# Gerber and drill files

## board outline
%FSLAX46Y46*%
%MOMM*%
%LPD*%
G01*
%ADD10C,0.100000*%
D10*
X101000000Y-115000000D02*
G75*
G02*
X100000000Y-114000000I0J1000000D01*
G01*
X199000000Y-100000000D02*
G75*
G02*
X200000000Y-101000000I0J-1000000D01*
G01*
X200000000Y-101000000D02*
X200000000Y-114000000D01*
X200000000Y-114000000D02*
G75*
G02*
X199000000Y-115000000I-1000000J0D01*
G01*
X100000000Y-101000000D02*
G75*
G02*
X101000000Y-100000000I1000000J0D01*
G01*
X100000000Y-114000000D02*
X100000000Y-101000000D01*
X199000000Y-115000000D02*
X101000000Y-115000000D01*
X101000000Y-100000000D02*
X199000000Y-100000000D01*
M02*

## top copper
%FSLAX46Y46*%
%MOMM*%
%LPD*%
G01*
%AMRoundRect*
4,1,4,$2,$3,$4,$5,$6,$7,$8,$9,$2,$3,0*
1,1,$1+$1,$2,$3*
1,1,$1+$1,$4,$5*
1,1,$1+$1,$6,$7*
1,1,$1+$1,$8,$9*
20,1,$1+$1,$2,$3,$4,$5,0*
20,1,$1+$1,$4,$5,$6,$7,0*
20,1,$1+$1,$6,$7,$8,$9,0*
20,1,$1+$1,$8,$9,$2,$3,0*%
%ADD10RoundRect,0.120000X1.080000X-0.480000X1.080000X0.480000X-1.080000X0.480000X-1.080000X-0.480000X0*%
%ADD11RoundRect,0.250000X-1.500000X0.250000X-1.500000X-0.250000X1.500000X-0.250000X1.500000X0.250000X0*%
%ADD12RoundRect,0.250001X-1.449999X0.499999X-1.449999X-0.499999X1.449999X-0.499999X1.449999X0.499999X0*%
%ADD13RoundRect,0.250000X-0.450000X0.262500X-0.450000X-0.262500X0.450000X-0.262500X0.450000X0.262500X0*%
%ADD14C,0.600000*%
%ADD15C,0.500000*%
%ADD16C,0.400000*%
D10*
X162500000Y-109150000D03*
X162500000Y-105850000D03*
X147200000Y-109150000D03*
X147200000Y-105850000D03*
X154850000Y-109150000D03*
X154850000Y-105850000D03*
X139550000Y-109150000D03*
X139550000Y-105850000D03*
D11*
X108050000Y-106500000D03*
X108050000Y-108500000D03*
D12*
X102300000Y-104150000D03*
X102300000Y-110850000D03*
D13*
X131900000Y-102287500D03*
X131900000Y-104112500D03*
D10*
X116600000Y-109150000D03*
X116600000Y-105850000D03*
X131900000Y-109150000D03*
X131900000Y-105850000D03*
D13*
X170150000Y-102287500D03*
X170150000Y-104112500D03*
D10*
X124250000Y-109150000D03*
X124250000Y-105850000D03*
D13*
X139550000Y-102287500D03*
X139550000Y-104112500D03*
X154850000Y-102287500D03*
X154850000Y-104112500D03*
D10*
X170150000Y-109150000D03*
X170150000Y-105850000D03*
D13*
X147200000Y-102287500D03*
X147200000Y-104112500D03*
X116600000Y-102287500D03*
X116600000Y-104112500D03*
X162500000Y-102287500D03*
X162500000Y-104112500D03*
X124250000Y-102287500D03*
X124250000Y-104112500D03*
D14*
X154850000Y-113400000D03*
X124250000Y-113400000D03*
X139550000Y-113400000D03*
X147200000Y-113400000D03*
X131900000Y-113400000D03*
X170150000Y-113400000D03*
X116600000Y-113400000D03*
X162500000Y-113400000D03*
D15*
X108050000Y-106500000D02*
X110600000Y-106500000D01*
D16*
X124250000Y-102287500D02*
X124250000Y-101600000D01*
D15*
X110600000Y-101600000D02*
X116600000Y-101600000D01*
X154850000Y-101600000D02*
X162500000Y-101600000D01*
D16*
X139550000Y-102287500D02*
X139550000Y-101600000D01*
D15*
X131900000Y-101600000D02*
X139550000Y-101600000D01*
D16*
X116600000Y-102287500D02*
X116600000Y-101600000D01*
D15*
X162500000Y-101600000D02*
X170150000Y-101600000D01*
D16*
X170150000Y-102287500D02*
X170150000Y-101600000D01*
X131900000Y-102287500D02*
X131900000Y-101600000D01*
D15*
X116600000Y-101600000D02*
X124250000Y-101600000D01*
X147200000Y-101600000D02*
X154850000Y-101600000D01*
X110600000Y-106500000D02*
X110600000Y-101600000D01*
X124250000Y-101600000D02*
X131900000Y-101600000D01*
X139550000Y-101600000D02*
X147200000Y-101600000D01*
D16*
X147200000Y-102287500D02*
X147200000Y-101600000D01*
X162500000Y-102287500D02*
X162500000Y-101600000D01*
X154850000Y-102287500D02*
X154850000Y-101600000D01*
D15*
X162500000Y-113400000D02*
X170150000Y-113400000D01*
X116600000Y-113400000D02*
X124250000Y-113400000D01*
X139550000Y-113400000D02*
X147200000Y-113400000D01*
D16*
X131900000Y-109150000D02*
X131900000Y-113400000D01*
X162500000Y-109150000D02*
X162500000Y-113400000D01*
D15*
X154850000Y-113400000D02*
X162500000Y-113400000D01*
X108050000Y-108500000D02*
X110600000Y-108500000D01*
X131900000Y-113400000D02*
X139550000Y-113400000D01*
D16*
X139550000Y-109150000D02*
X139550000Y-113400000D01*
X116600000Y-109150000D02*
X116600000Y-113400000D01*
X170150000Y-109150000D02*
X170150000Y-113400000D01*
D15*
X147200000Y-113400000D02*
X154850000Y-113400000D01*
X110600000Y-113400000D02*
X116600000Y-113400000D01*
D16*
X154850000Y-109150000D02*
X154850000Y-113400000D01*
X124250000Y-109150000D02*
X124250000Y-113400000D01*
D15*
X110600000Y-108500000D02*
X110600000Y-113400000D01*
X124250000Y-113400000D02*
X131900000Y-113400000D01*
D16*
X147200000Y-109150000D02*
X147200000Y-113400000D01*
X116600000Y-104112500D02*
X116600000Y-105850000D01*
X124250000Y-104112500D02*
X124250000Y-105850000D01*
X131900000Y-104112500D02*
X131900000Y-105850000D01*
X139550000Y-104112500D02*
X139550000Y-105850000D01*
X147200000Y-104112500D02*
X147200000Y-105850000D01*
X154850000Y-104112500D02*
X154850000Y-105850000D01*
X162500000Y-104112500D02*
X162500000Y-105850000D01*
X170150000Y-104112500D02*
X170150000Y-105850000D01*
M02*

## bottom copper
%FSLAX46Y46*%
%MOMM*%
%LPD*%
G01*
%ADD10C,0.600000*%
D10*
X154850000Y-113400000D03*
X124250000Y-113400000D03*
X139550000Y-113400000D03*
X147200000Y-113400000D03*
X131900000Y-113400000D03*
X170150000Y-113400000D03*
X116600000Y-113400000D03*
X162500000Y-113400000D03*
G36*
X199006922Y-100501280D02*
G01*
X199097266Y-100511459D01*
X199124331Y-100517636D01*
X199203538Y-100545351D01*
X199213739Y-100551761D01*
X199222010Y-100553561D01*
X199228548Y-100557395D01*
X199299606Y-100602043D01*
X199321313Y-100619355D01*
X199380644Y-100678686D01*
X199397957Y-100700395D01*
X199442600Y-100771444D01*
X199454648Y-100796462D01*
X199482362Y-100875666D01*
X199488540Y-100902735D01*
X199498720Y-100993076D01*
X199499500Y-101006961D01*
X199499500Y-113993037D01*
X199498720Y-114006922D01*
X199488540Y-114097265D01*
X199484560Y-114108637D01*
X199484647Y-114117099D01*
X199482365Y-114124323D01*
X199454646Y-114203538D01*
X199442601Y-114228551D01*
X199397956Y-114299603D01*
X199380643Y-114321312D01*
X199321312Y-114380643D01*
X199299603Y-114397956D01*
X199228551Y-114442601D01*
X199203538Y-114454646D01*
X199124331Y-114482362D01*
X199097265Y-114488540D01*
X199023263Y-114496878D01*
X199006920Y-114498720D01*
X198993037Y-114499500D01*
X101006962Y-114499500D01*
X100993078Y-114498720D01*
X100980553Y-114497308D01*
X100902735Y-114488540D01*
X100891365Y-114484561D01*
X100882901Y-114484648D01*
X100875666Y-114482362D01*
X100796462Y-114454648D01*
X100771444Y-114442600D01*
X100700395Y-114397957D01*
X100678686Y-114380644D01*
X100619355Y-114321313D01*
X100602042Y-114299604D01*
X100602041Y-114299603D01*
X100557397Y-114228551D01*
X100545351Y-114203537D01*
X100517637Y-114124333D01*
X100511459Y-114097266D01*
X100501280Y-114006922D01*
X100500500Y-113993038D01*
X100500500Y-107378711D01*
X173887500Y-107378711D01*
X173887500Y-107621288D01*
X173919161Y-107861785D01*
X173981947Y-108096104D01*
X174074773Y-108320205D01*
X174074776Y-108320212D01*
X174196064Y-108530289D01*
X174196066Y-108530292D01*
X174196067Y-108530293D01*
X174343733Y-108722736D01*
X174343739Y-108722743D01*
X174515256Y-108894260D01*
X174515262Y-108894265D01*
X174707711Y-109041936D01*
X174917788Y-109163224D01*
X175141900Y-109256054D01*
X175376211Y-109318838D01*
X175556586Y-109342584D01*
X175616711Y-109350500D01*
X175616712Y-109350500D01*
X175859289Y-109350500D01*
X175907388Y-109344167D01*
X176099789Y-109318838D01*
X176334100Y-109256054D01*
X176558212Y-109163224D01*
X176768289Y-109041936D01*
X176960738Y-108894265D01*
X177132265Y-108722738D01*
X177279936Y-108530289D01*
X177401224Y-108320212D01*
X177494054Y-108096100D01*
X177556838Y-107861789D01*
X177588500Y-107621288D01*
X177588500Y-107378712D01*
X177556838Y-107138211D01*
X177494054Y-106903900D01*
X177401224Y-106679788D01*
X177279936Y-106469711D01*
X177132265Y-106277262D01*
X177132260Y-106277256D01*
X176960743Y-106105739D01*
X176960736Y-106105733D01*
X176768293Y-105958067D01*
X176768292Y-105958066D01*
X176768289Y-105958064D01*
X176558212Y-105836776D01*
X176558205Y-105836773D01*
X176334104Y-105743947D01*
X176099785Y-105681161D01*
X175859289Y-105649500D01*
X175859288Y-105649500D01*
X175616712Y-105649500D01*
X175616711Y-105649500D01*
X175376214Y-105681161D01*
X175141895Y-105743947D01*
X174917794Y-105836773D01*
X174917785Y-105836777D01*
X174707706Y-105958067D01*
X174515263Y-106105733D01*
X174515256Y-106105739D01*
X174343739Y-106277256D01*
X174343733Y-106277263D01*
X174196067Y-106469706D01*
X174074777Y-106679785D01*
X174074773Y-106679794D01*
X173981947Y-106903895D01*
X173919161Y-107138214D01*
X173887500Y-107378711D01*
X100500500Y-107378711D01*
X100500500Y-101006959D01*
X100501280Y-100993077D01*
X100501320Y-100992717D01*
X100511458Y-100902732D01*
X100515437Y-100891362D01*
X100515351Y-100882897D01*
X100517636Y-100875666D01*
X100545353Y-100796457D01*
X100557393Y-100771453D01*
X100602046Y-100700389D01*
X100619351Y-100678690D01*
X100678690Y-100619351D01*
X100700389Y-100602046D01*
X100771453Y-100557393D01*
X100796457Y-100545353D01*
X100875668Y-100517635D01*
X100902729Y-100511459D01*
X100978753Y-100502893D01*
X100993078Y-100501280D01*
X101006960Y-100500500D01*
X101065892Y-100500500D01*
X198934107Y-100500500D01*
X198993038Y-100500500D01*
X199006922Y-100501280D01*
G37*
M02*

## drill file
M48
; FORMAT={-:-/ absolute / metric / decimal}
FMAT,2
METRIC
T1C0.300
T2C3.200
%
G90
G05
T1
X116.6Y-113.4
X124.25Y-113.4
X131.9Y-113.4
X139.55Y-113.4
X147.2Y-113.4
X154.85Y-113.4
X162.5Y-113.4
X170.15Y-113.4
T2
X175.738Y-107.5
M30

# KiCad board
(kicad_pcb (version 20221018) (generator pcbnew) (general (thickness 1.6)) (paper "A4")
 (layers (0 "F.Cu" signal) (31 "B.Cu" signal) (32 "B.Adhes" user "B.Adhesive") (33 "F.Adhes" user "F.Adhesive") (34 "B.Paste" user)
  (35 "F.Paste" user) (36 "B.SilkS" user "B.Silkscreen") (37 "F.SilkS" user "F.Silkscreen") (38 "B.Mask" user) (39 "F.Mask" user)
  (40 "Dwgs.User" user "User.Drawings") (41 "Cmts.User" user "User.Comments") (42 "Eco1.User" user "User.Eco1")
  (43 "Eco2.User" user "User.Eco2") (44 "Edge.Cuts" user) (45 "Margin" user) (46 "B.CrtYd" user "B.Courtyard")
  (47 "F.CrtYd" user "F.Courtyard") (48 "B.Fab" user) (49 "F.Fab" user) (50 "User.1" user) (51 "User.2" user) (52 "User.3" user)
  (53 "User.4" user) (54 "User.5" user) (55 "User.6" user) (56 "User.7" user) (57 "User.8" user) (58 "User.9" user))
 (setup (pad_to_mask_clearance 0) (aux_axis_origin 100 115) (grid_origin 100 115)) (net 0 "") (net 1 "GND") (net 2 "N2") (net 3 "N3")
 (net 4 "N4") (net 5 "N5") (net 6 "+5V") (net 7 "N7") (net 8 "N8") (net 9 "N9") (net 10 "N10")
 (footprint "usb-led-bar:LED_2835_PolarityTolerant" (layer "F.Cu") (at 162.5 107.5 90)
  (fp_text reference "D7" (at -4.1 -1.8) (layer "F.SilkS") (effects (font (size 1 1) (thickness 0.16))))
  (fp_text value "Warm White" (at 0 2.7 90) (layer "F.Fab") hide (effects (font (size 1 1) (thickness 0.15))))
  (pad "1" smd roundrect (at -1.65 0 90) (size 1.2 2.4) (layers "F.Cu" "F.Paste" "F.Mask") (roundrect_rratio 0.1) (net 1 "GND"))
  (pad "2" smd roundrect (at 1.65 0 90) (size 1.2 2.4) (layers "F.Cu" "F.Paste" "F.Mask") (roundrect_rratio 0.1) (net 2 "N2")))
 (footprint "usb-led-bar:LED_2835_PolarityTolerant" (layer "F.Cu") (at 147.2 107.5 90)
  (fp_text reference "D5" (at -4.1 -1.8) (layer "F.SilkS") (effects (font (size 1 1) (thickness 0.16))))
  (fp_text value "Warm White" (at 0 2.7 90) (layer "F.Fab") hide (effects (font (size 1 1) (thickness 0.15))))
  (pad "1" smd roundrect (at -1.65 0 90) (size 1.2 2.4) (layers "F.Cu" "F.Paste" "F.Mask") (roundrect_rratio 0.1) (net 1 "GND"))
  (pad "2" smd roundrect (at 1.65 0 90) (size 1.2 2.4) (layers "F.Cu" "F.Paste" "F.Mask") (roundrect_rratio 0.1) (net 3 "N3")))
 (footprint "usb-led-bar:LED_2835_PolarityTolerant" (layer "F.Cu") (at 154.85 107.5 90)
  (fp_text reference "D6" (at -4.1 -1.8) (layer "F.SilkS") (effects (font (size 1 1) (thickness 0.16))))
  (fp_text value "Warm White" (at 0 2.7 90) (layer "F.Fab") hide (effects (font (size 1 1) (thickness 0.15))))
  (pad "1" smd roundrect (at -1.65 0 90) (size 1.2 2.4) (layers "F.Cu" "F.Paste" "F.Mask") (roundrect_rratio 0.1) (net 1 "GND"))
  (pad "2" smd roundrect (at 1.65 0 90) (size 1.2 2.4) (layers "F.Cu" "F.Paste" "F.Mask") (roundrect_rratio 0.1) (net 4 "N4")))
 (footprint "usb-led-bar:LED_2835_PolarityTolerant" (layer "F.Cu") (at 139.55 107.5 90)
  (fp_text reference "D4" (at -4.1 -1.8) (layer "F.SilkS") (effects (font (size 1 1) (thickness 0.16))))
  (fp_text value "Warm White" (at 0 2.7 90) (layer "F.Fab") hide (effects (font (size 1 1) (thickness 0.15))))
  (pad "1" smd roundrect (at -1.65 0 90) (size 1.2 2.4) (layers "F.Cu" "F.Paste" "F.Mask") (roundrect_rratio 0.1) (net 1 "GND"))
  (pad "2" smd roundrect (at 1.65 0 90) (size 1.2 2.4) (layers "F.Cu" "F.Paste" "F.Mask") (roundrect_rratio 0.1) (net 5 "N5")))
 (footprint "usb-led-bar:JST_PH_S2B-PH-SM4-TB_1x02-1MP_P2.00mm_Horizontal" (layer "F.Cu") (at 105.2 107.5 -90)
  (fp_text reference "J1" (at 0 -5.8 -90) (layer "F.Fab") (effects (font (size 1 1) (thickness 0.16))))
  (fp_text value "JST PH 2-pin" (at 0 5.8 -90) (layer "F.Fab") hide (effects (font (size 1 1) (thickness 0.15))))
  (pad "1" smd roundrect (at -1 -2.85 270) (size 1 3.5) (layers "F.Cu" "F.Paste" "F.Mask") (roundrect_rratio 0.25) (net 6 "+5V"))
  (pad "2" smd roundrect (at 1 -2.85 270) (size 1 3.5) (layers "F.Cu" "F.Paste" "F.Mask") (roundrect_rratio 0.25) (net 1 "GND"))
  (pad "MP" smd roundrect (at -3.35 2.9 270) (size 1.5 3.4) (layers "F.Cu" "F.Paste" "F.Mask") (roundrect_rratio 0.166667))
  (pad "MP" smd roundrect (at 3.35 2.9 270) (size 1.5 3.4) (layers "F.Cu" "F.Paste" "F.Mask") (roundrect_rratio 0.166667)))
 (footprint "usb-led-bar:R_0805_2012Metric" (layer "F.Cu") (at 131.9 103.2 -90)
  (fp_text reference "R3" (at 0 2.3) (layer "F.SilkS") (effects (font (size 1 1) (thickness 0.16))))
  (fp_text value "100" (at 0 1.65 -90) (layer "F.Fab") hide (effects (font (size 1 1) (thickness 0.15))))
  (pad "1" smd roundrect (at -0.9125 0 270) (size 1.025 1.4) (layers "F.Cu" "F.Paste" "F.Mask") (roundrect_rratio 0.243902) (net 6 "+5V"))
  (pad "2" smd roundrect (at 0.9125 0 270) (size 1.025 1.4) (layers "F.Cu" "F.Paste" "F.Mask") (roundrect_rratio 0.243902) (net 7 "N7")))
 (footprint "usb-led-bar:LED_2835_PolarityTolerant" (layer "F.Cu") (at 116.6 107.5 90)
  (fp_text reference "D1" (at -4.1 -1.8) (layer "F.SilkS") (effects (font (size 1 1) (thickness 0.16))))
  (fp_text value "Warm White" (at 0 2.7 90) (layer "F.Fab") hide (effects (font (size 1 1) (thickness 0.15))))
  (pad "1" smd roundrect (at -1.65 0 90) (size 1.2 2.4) (layers "F.Cu" "F.Paste" "F.Mask") (roundrect_rratio 0.1) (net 1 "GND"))
  (pad "2" smd roundrect (at 1.65 0 90) (size 1.2 2.4) (layers "F.Cu" "F.Paste" "F.Mask") (roundrect_rratio 0.1) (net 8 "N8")))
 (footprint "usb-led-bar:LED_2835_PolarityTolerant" (layer "F.Cu") (at 131.9 107.5 90)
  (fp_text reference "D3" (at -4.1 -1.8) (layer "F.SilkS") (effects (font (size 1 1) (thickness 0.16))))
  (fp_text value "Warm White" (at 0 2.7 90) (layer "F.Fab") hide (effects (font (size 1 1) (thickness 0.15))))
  (pad "1" smd roundrect (at -1.65 0 90) (size 1.2 2.4) (layers "F.Cu" "F.Paste" "F.Mask") (roundrect_rratio 0.1) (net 1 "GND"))
  (pad "2" smd roundrect (at 1.65 0 90) (size 1.2 2.4) (layers "F.Cu" "F.Paste" "F.Mask") (roundrect_rratio 0.1) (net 7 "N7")))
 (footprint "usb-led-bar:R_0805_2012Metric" (layer "F.Cu") (at 170.15 103.2 -90)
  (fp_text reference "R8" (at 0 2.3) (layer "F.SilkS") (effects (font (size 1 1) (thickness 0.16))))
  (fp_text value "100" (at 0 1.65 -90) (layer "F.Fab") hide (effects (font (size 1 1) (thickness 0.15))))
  (pad "1" smd roundrect (at -0.9125 0 270) (size 1.025 1.4) (layers "F.Cu" "F.Paste" "F.Mask") (roundrect_rratio 0.243902) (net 6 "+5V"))
  (pad "2" smd roundrect (at 0.9125 0 270) (size 1.025 1.4) (layers "F.Cu" "F.Paste" "F.Mask") (roundrect_rratio 0.243902) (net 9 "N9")))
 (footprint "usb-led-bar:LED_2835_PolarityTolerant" (layer "F.Cu") (at 124.25 107.5 90)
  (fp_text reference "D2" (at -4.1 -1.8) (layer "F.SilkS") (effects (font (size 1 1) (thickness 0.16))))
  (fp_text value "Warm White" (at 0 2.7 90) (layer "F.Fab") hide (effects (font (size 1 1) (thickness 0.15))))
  (pad "1" smd roundrect (at -1.65 0 90) (size 1.2 2.4) (layers "F.Cu" "F.Paste" "F.Mask") (roundrect_rratio 0.1) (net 1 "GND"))
  (pad "2" smd roundrect (at 1.65 0 90) (size 1.2 2.4) (layers "F.Cu" "F.Paste" "F.Mask") (roundrect_rratio 0.1) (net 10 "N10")))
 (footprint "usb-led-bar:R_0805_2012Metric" (layer "F.Cu") (at 139.55 103.2 -90)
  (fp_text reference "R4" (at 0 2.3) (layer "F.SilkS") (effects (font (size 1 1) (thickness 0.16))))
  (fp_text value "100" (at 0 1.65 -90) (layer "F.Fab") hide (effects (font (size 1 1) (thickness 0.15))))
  (pad "1" smd roundrect (at -0.9125 0 270) (size 1.025 1.4) (layers "F.Cu" "F.Paste" "F.Mask") (roundrect_rratio 0.243902) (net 6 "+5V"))
  (pad "2" smd roundrect (at 0.9125 0 270) (size 1.025 1.4) (layers "F.Cu" "F.Paste" "F.Mask") (roundrect_rratio 0.243902) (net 5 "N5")))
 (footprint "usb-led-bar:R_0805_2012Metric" (layer "F.Cu") (at 154.85 103.2 -90)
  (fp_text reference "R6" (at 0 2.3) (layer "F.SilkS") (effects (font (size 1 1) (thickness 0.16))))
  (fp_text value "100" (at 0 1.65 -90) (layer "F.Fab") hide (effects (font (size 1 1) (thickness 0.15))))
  (pad "1" smd roundrect (at -0.9125 0 270) (size 1.025 1.4) (layers "F.Cu" "F.Paste" "F.Mask") (roundrect_rratio 0.243902) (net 6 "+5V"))
  (pad "2" smd roundrect (at 0.9125 0 270) (size 1.025 1.4) (layers "F.Cu" "F.Paste" "F.Mask") (roundrect_rratio 0.243902) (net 4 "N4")))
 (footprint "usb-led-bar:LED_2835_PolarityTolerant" (layer "F.Cu") (at 170.15 107.5 90)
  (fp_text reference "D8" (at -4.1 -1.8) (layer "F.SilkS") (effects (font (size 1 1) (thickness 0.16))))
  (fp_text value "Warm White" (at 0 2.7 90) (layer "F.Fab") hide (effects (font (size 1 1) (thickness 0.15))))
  (pad "1" smd roundrect (at -1.65 0 90) (size 1.2 2.4) (layers "F.Cu" "F.Paste" "F.Mask") (roundrect_rratio 0.1) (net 1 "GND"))
  (pad "2" smd roundrect (at 1.65 0 90) (size 1.2 2.4) (layers "F.Cu" "F.Paste" "F.Mask") (roundrect_rratio 0.1) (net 9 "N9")))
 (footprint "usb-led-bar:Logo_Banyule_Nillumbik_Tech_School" (layer "F.Cu") (at 189.244 107.5)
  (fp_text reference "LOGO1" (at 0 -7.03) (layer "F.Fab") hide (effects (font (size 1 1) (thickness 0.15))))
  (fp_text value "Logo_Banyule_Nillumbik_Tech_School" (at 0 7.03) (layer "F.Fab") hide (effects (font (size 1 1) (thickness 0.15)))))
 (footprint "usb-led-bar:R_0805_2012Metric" (layer "F.Cu") (at 147.2 103.2 -90)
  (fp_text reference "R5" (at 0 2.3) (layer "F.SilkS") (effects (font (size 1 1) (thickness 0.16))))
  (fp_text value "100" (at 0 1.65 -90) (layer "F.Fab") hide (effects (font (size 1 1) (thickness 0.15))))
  (pad "1" smd roundrect (at -0.9125 0 270) (size 1.025 1.4) (layers "F.Cu" "F.Paste" "F.Mask") (roundrect_rratio 0.243902) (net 6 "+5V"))
  (pad "2" smd roundrect (at 0.9125 0 270) (size 1.025 1.4) (layers "F.Cu" "F.Paste" "F.Mask") (roundrect_rratio 0.243902) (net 3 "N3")))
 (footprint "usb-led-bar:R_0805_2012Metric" (layer "F.Cu") (at 116.6 103.2 -90)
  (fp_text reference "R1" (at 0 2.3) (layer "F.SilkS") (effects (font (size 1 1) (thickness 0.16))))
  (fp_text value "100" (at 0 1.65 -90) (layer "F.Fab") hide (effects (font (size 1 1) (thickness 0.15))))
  (pad "1" smd roundrect (at -0.9125 0 270) (size 1.025 1.4) (layers "F.Cu" "F.Paste" "F.Mask") (roundrect_rratio 0.243902) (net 6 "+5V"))
  (pad "2" smd roundrect (at 0.9125 0 270) (size 1.025 1.4) (layers "F.Cu" "F.Paste" "F.Mask") (roundrect_rratio 0.243902) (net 8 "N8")))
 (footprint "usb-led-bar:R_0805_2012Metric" (layer "F.Cu") (at 162.5 103.2 -90)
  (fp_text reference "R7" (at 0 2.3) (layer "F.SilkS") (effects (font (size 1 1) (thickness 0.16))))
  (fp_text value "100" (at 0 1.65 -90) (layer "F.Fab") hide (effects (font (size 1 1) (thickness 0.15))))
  (pad "1" smd roundrect (at -0.9125 0 270) (size 1.025 1.4) (layers "F.Cu" "F.Paste" "F.Mask") (roundrect_rratio 0.243902) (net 6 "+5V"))
  (pad "2" smd roundrect (at 0.9125 0 270) (size 1.025 1.4) (layers "F.Cu" "F.Paste" "F.Mask") (roundrect_rratio 0.243902) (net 2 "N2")))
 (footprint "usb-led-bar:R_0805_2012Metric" (layer "F.Cu") (at 124.25 103.2 -90)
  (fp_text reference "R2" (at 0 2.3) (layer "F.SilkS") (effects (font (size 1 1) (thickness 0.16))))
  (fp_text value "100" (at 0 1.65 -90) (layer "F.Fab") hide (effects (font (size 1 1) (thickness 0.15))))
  (pad "1" smd roundrect (at -0.9125 0 270) (size 1.025 1.4) (layers "F.Cu" "F.Paste" "F.Mask") (roundrect_rratio 0.243902) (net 6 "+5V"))
  (pad "2" smd roundrect (at 0.9125 0 270) (size 1.025 1.4) (layers "F.Cu" "F.Paste" "F.Mask") (roundrect_rratio 0.243902) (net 10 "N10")))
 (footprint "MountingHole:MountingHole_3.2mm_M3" (layer "F.Cu") (at 175.738 107.5)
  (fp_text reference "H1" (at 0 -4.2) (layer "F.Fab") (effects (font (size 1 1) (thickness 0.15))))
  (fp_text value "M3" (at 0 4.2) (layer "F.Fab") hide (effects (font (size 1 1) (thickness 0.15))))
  (pad "" np_thru_hole circle (at 0 0) (size 3.2 3.2) (drill 3.2) (layers "*.Cu" "*.Mask")))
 (gr_arc (start 101 115) (mid 100.292893 114.707106) (end 100 114) (stroke (width 0.1) (type default)) (layer "Edge.Cuts"))
 (gr_arc (start 199 100) (mid 199.707106 100.292893) (end 200 101) (stroke (width 0.1) (type default)) (layer "Edge.Cuts"))
 (gr_line (start 200 101) (end 200 114) (stroke (width 0.1) (type default)) (layer "Edge.Cuts"))
 (gr_arc (start 200 114) (mid 199.707106 114.707106) (end 199 115) (stroke (width 0.1) (type default)) (layer "Edge.Cuts"))
 (gr_arc (start 100 101) (mid 100.292893 100.292893) (end 101 100) (stroke (width 0.1) (type default)) (layer "Edge.Cuts"))
 (gr_line (start 100 114) (end 100 101) (stroke (width 0.1) (type default)) (layer "Edge.Cuts"))
 (gr_line (start 199 115) (end 101 115) (stroke (width 0.1) (type default)) (layer "Edge.Cuts"))
 (gr_line (start 101 100) (end 199 100) (stroke (width 0.1) (type default)) (layer "Edge.Cuts"))
 (segment (start 108.05 106.5) (end 110.6 106.5) (width 0.5) (layer "F.Cu") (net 6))
 (segment (start 124.25 102.2875) (end 124.25 101.6) (width 0.4) (layer "F.Cu") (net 6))
 (segment (start 110.6 101.6) (end 116.6 101.6) (width 0.5) (layer "F.Cu") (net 6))
 (segment (start 154.85 101.6) (end 162.5 101.6) (width 0.5) (layer "F.Cu") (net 6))
 (segment (start 139.55 102.2875) (end 139.55 101.6) (width 0.4) (layer "F.Cu") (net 6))
 (segment (start 131.9 101.6) (end 139.55 101.6) (width 0.5) (layer "F.Cu") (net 6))
 (segment (start 116.6 102.2875) (end 116.6 101.6) (width 0.4) (layer "F.Cu") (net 6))
 (segment (start 162.5 101.6) (end 170.15 101.6) (width 0.5) (layer "F.Cu") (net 6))
 (segment (start 170.15 102.2875) (end 170.15 101.6) (width 0.4) (layer "F.Cu") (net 6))
 (segment (start 131.9 102.2875) (end 131.9 101.6) (width 0.4) (layer "F.Cu") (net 6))
 (segment (start 116.6 101.6) (end 124.25 101.6) (width 0.5) (layer "F.Cu") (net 6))
 (segment (start 147.2 101.6) (end 154.85 101.6) (width 0.5) (layer "F.Cu") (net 6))
 (segment (start 110.6 106.5) (end 110.6 101.6) (width 0.5) (layer "F.Cu") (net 6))
 (segment (start 124.25 101.6) (end 131.9 101.6) (width 0.5) (layer "F.Cu") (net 6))
 (segment (start 139.55 101.6) (end 147.2 101.6) (width 0.5) (layer "F.Cu") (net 6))
 (segment (start 147.2 102.2875) (end 147.2 101.6) (width 0.4) (layer "F.Cu") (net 6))
 (segment (start 162.5 102.2875) (end 162.5 101.6) (width 0.4) (layer "F.Cu") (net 6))
 (segment (start 154.85 102.2875) (end 154.85 101.6) (width 0.4) (layer "F.Cu") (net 6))
 (segment (start 162.5 113.4) (end 170.15 113.4) (width 0.5) (layer "F.Cu") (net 1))
 (segment (start 116.6 113.4) (end 124.25 113.4) (width 0.5) (layer "F.Cu") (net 1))
 (segment (start 139.55 113.4) (end 147.2 113.4) (width 0.5) (layer "F.Cu") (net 1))
 (segment (start 131.9 109.15) (end 131.9 113.4) (width 0.4) (layer "F.Cu") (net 1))
 (segment (start 162.5 109.15) (end 162.5 113.4) (width 0.4) (layer "F.Cu") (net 1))
 (segment (start 154.85 113.4) (end 162.5 113.4) (width 0.5) (layer "F.Cu") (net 1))
 (segment (start 108.05 108.5) (end 110.6 108.5) (width 0.5) (layer "F.Cu") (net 1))
 (segment (start 131.9 113.4) (end 139.55 113.4) (width 0.5) (layer "F.Cu") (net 1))
 (segment (start 139.55 109.15) (end 139.55 113.4) (width 0.4) (layer "F.Cu") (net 1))
 (segment (start 116.6 109.15) (end 116.6 113.4) (width 0.4) (layer "F.Cu") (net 1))
 (segment (start 170.15 109.15) (end 170.15 113.4) (width 0.4) (layer "F.Cu") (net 1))
 (segment (start 147.2 113.4) (end 154.85 113.4) (width 0.5) (layer "F.Cu") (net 1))
 (segment (start 110.6 113.4) (end 116.6 113.4) (width 0.5) (layer "F.Cu") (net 1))
 (segment (start 154.85 109.15) (end 154.85 113.4) (width 0.4) (layer "F.Cu") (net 1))
 (segment (start 124.25 109.15) (end 124.25 113.4) (width 0.4) (layer "F.Cu") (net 1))
 (segment (start 110.6 108.5) (end 110.6 113.4) (width 0.5) (layer "F.Cu") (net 1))
 (segment (start 124.25 113.4) (end 131.9 113.4) (width 0.5) (layer "F.Cu") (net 1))
 (segment (start 147.2 109.15) (end 147.2 113.4) (width 0.4) (layer "F.Cu") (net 1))
 (via (at 154.85 113.4) (size 0.6) (drill 0.3) (layers "F.Cu" "B.Cu") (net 1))
 (via (at 124.25 113.4) (size 0.6) (drill 0.3) (layers "F.Cu" "B.Cu") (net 1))
 (via (at 139.55 113.4) (size 0.6) (drill 0.3) (layers "F.Cu" "B.Cu") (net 1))
 (via (at 147.2 113.4) (size 0.6) (drill 0.3) (layers "F.Cu" "B.Cu") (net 1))
 (via (at 131.9 113.4) (size 0.6) (drill 0.3) (layers "F.Cu" "B.Cu") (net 1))
 (via (at 170.15 113.4) (size 0.6) (drill 0.3) (layers "F.Cu" "B.Cu") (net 1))
 (via (at 116.6 113.4) (size 0.6) (drill 0.3) (layers "F.Cu" "B.Cu") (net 1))
 (via (at 162.5 113.4) (size 0.6) (drill 0.3) (layers "F.Cu" "B.Cu") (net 1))
 (segment (start 116.6 104.1125) (end 116.6 105.85) (width 0.4) (layer "F.Cu") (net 8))
 (segment (start 124.25 104.1125) (end 124.25 105.85) (width 0.4) (layer "F.Cu") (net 10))
 (segment (start 131.9 104.1125) (end 131.9 105.85) (width 0.4) (layer "F.Cu") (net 7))
 (segment (start 139.55 104.1125) (end 139.55 105.85) (width 0.4) (layer "F.Cu") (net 5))
 (segment (start 147.2 104.1125) (end 147.2 105.85) (width 0.4) (layer "F.Cu") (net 3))
 (segment (start 154.85 104.1125) (end 154.85 105.85) (width 0.4) (layer "F.Cu") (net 4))
 (segment (start 162.5 104.1125) (end 162.5 105.85) (width 0.4) (layer "F.Cu") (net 2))
 (segment (start 170.15 104.1125) (end 170.15 105.85) (width 0.4) (layer "F.Cu") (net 9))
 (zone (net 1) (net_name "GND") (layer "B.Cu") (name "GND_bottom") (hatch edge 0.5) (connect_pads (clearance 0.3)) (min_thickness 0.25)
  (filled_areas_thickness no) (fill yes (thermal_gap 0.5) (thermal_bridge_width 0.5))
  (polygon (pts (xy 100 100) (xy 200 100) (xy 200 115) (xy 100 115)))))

